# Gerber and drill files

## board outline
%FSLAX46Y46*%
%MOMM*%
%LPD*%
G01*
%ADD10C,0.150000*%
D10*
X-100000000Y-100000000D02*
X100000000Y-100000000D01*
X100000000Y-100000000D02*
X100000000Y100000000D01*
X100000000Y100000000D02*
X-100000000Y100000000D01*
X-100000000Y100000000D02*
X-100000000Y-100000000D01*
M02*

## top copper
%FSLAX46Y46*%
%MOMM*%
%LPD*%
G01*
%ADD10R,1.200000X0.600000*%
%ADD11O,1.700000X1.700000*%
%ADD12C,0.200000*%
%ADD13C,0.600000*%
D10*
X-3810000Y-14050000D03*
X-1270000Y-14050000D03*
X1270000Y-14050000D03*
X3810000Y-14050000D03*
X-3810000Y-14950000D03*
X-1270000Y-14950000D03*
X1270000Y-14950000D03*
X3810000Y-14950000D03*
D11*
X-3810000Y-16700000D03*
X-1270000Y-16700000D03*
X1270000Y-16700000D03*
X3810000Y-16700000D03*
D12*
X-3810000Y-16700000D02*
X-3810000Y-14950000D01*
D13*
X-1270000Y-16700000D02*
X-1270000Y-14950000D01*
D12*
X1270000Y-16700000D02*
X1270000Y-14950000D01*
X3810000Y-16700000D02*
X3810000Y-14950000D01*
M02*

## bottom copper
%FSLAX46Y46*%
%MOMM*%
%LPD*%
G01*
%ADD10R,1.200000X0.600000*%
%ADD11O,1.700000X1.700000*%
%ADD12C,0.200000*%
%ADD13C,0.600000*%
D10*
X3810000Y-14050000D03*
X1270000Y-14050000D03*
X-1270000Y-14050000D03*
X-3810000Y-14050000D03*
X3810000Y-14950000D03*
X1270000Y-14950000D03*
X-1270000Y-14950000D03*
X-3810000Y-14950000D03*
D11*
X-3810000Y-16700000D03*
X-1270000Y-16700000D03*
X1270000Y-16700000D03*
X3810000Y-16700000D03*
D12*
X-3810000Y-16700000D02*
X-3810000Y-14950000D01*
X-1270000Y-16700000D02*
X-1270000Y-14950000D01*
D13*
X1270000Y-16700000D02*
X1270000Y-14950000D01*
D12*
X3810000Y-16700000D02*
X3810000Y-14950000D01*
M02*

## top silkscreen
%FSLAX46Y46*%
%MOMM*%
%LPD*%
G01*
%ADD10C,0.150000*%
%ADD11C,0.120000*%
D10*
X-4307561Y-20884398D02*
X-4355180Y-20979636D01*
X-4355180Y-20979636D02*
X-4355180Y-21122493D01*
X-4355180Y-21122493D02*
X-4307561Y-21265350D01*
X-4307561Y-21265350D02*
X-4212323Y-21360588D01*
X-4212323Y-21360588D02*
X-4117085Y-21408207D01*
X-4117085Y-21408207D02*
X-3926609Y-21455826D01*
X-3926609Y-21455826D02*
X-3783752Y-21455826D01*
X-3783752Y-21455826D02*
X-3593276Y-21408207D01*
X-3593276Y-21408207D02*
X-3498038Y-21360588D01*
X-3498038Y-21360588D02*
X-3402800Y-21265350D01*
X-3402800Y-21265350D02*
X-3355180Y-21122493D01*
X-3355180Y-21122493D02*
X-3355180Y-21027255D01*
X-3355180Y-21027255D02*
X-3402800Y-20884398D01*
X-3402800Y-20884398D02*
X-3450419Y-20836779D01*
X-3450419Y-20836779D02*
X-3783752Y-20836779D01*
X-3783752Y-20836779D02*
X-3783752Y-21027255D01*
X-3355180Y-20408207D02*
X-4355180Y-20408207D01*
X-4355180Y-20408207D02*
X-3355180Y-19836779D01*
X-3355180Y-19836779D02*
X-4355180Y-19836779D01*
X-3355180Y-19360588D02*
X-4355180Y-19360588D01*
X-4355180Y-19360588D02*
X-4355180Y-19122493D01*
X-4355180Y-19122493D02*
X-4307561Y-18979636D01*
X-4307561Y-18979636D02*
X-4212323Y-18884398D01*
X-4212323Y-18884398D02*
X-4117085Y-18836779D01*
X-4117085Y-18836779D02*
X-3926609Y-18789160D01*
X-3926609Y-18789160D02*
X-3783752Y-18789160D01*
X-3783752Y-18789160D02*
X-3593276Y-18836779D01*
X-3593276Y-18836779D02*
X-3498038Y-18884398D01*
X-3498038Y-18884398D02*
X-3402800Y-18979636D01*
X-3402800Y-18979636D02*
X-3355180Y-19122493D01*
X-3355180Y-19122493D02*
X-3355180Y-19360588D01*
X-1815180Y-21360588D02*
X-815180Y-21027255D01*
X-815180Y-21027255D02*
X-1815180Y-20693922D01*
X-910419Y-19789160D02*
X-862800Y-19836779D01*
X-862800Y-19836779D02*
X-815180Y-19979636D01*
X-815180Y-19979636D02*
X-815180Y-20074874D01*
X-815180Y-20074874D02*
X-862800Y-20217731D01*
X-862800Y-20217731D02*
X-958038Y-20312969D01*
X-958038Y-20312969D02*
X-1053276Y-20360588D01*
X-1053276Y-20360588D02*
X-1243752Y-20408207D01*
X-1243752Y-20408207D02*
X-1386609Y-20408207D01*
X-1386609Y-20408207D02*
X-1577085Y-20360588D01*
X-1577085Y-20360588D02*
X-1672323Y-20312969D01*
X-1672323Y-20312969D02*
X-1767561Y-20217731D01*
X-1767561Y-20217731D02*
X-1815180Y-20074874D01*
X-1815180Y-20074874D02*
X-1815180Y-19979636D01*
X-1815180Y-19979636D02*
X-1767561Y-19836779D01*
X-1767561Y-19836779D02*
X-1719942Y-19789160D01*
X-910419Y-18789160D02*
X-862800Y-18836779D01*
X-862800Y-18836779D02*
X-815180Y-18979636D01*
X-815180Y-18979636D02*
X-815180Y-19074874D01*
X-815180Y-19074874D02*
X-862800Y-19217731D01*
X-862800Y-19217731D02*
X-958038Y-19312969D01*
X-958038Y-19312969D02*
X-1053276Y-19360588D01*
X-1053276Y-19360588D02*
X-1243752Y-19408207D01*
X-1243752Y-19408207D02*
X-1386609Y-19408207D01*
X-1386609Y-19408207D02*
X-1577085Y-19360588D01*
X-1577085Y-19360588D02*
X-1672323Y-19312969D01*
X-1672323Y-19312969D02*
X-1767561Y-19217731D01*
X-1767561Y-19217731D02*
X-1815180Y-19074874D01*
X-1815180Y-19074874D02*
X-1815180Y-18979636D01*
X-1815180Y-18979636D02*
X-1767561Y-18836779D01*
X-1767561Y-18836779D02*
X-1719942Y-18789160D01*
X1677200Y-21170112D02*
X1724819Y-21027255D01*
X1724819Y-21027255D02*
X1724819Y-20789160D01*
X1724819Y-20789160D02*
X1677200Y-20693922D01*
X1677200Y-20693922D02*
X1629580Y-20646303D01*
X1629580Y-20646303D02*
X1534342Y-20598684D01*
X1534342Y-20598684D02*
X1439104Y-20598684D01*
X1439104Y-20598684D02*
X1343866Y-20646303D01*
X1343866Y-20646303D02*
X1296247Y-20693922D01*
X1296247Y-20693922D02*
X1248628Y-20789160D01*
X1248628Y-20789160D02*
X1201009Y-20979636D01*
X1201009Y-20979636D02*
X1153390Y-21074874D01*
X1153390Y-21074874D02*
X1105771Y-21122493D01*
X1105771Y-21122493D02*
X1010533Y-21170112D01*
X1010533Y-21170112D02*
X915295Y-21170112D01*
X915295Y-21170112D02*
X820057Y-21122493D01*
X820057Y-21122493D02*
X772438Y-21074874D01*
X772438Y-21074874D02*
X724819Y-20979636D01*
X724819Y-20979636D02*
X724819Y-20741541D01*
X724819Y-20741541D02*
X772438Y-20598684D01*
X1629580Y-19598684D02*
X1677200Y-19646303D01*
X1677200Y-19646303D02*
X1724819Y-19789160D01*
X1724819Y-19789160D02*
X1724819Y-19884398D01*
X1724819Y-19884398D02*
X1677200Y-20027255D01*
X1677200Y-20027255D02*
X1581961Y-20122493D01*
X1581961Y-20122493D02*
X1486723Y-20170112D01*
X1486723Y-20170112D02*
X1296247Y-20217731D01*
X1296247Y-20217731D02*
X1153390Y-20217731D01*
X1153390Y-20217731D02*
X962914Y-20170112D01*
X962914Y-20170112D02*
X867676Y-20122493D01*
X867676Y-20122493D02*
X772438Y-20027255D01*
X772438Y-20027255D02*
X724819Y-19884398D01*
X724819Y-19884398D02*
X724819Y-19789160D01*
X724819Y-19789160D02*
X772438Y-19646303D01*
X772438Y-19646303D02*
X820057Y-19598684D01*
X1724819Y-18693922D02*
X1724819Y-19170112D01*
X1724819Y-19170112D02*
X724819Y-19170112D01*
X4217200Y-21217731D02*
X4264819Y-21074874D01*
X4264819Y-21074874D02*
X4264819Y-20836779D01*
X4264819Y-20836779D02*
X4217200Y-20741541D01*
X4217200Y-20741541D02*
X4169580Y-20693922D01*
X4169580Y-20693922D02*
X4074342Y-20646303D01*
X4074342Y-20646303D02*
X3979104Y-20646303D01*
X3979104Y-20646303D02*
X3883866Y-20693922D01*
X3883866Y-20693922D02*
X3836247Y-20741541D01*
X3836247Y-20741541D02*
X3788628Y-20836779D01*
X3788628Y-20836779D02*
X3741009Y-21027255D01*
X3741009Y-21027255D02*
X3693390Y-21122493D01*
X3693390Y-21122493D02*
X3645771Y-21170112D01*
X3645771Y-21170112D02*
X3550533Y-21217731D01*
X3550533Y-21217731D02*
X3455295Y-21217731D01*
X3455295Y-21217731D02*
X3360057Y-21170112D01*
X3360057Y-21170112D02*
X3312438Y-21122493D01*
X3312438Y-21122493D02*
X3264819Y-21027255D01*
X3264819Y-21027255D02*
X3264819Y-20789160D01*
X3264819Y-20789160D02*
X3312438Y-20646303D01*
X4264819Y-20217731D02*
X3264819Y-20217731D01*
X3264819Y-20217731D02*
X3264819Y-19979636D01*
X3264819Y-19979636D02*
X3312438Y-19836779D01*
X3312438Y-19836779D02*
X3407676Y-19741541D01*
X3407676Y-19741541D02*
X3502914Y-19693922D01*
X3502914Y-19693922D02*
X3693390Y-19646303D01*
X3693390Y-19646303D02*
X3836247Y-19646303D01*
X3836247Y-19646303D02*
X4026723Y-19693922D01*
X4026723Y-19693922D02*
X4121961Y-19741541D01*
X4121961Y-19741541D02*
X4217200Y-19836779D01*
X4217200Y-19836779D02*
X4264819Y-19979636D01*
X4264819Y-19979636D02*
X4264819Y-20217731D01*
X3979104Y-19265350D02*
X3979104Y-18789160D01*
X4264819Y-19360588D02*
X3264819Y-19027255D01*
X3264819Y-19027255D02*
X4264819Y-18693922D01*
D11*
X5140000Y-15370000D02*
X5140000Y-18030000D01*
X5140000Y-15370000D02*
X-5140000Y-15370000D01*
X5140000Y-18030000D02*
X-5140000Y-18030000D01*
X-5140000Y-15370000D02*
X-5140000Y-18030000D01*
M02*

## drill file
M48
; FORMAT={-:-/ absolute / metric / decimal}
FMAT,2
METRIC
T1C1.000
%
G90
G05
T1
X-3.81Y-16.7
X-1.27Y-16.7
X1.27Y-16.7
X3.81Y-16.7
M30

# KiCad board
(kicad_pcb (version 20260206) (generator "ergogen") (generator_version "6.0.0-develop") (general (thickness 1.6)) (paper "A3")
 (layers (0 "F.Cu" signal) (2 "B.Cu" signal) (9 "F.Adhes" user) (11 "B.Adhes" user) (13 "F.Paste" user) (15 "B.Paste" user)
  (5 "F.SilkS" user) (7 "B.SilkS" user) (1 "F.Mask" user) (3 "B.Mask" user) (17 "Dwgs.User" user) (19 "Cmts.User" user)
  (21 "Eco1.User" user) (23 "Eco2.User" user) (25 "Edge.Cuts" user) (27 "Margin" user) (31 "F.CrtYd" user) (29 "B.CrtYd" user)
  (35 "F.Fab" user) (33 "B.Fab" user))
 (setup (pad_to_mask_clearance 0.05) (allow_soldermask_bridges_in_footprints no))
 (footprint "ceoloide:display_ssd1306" (layer "F.Cu") (at 0 0 0)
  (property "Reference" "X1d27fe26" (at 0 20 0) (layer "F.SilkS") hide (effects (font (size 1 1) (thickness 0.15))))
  (fp_line (start 5.14 15.37) (end 5.14 18.03) (layer "F.SilkS") (stroke (width 0.12) (type solid)))
  (fp_line (start 5.14 15.37) (end -5.14 15.37) (layer "F.SilkS") (stroke (width 0.12) (type solid)))
  (fp_line (start 5.14 18.03) (end -5.14 18.03) (layer "F.SilkS") (stroke (width 0.12) (type solid)))
  (fp_line (start -5.14 15.37) (end -5.14 18.03) (layer "F.SilkS") (stroke (width 0.12) (type solid)))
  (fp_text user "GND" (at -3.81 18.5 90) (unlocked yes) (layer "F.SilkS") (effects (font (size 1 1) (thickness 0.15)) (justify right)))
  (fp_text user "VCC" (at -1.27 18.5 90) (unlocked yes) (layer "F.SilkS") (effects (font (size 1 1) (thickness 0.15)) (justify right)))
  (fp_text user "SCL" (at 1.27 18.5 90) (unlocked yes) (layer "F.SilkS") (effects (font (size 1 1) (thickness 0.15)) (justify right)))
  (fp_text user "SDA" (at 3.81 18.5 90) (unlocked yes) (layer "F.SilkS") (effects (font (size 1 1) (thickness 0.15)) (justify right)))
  (pad "14" smd rect (at -3.81 14.05 90) (size 0.6 1.2) (layers "F.Cu" "F.Paste" "F.Mask") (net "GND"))
  (pad "15" smd rect (at -1.27 14.05 90) (size 0.6 1.2) (layers "F.Cu" "F.Paste" "F.Mask") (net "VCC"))
  (pad "16" smd rect (at 1.27 14.05 90) (size 0.6 1.2) (layers "F.Cu" "F.Paste" "F.Mask") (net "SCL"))
  (pad "17" smd rect (at 3.81 14.05 90) (size 0.6 1.2) (layers "F.Cu" "F.Paste" "F.Mask") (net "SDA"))
  (pad "10" smd rect (at -3.81 14.95 90) (size 0.6 1.2) (layers "F.Cu" "F.Paste" "F.Mask") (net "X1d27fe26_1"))
  (pad "11" smd rect (at -1.27 14.95 90) (size 0.6 1.2) (layers "F.Cu" "F.Paste" "F.Mask") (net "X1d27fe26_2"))
  (pad "12" smd rect (at 1.27 14.95 90) (size 0.6 1.2) (layers "F.Cu" "F.Paste" "F.Mask") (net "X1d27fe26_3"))
  (pad "13" smd rect (at 3.81 14.95 90) (size 0.6 1.2) (layers "F.Cu" "F.Paste" "F.Mask") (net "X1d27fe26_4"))
  (pad "24" smd rect (at 3.81 14.05 270) (size 0.6 1.2) (layers "B.Cu" "B.Paste" "B.Mask") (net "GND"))
  (pad "25" smd rect (at 1.27 14.05 270) (size 0.6 1.2) (layers "B.Cu" "B.Paste" "B.Mask") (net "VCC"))
  (pad "26" smd rect (at -1.27 14.05 270) (size 0.6 1.2) (layers "B.Cu" "B.Paste" "B.Mask") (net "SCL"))
  (pad "27" smd rect (at -3.81 14.05 270) (size 0.6 1.2) (layers "B.Cu" "B.Paste" "B.Mask") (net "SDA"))
  (pad "20" smd rect (at 3.81 14.95 270) (size 0.6 1.2) (layers "B.Cu" "B.Paste" "B.Mask") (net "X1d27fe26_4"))
  (pad "21" smd rect (at 1.27 14.95 270) (size 0.6 1.2) (layers "B.Cu" "B.Paste" "B.Mask") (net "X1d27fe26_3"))
  (pad "22" smd rect (at -1.27 14.95 270) (size 0.6 1.2) (layers "B.Cu" "B.Paste" "B.Mask") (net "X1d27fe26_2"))
  (pad "23" smd rect (at -3.81 14.95 270) (size 0.6 1.2) (layers "B.Cu" "B.Paste" "B.Mask") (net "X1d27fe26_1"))
  (pad "1" thru_hole oval (at -3.81 16.7 270) (size 1.7 1.7) (drill 1) (layers "*.Cu" "*.Mask") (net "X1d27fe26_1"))
  (pad "2" thru_hole oval (at -1.27 16.7 270) (size 1.7 1.7) (drill 1) (layers "*.Cu" "*.Mask") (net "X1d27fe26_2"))
  (pad "3" thru_hole oval (at 1.27 16.7 270) (size 1.7 1.7) (drill 1) (layers "*.Cu" "*.Mask") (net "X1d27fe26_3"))
  (pad "4" thru_hole oval (at 3.81 16.7 270) (size 1.7 1.7) (drill 1) (layers "*.Cu" "*.Mask") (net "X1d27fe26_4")))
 (segment (start -3.81 16.7) (end -3.81 14.95) (width 0.2) (layer "F.Cu") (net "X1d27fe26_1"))
 (segment (start -1.27 16.7) (end -1.27 14.95) (width 0.6) (layer "F.Cu") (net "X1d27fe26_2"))
 (segment (start 1.27 16.7) (end 1.27 14.95) (width 0.2) (layer "F.Cu") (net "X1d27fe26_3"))
 (segment (start 3.81 16.7) (end 3.81 14.95) (width 0.2) (layer "F.Cu") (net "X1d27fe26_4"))
 (segment (start -3.81 16.7) (end -3.81 14.95) (width 0.2) (layer "B.Cu") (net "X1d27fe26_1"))
 (segment (start -1.27 16.7) (end -1.27 14.95) (width 0.2) (layer "B.Cu") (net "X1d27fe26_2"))
 (segment (start 1.27 16.7) (end 1.27 14.95) (width 0.6) (layer "B.Cu") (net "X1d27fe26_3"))
 (segment (start 3.81 16.7) (end 3.81 14.95) (width 0.2) (layer "B.Cu") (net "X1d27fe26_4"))
 (gr_line (start -100 100) (end 100 100) (layer Edge.Cuts) (stroke (width 0.15) (type default)))
 (gr_line (start 100 100) (end 100 -100) (layer Edge.Cuts) (stroke (width 0.15) (type default)))
 (gr_line (start 100 -100) (end -100 -100) (layer Edge.Cuts) (stroke (width 0.15) (type default)))
 (gr_line (start -100 -100) (end -100 100) (layer Edge.Cuts) (stroke (width 0.15) (type default))))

